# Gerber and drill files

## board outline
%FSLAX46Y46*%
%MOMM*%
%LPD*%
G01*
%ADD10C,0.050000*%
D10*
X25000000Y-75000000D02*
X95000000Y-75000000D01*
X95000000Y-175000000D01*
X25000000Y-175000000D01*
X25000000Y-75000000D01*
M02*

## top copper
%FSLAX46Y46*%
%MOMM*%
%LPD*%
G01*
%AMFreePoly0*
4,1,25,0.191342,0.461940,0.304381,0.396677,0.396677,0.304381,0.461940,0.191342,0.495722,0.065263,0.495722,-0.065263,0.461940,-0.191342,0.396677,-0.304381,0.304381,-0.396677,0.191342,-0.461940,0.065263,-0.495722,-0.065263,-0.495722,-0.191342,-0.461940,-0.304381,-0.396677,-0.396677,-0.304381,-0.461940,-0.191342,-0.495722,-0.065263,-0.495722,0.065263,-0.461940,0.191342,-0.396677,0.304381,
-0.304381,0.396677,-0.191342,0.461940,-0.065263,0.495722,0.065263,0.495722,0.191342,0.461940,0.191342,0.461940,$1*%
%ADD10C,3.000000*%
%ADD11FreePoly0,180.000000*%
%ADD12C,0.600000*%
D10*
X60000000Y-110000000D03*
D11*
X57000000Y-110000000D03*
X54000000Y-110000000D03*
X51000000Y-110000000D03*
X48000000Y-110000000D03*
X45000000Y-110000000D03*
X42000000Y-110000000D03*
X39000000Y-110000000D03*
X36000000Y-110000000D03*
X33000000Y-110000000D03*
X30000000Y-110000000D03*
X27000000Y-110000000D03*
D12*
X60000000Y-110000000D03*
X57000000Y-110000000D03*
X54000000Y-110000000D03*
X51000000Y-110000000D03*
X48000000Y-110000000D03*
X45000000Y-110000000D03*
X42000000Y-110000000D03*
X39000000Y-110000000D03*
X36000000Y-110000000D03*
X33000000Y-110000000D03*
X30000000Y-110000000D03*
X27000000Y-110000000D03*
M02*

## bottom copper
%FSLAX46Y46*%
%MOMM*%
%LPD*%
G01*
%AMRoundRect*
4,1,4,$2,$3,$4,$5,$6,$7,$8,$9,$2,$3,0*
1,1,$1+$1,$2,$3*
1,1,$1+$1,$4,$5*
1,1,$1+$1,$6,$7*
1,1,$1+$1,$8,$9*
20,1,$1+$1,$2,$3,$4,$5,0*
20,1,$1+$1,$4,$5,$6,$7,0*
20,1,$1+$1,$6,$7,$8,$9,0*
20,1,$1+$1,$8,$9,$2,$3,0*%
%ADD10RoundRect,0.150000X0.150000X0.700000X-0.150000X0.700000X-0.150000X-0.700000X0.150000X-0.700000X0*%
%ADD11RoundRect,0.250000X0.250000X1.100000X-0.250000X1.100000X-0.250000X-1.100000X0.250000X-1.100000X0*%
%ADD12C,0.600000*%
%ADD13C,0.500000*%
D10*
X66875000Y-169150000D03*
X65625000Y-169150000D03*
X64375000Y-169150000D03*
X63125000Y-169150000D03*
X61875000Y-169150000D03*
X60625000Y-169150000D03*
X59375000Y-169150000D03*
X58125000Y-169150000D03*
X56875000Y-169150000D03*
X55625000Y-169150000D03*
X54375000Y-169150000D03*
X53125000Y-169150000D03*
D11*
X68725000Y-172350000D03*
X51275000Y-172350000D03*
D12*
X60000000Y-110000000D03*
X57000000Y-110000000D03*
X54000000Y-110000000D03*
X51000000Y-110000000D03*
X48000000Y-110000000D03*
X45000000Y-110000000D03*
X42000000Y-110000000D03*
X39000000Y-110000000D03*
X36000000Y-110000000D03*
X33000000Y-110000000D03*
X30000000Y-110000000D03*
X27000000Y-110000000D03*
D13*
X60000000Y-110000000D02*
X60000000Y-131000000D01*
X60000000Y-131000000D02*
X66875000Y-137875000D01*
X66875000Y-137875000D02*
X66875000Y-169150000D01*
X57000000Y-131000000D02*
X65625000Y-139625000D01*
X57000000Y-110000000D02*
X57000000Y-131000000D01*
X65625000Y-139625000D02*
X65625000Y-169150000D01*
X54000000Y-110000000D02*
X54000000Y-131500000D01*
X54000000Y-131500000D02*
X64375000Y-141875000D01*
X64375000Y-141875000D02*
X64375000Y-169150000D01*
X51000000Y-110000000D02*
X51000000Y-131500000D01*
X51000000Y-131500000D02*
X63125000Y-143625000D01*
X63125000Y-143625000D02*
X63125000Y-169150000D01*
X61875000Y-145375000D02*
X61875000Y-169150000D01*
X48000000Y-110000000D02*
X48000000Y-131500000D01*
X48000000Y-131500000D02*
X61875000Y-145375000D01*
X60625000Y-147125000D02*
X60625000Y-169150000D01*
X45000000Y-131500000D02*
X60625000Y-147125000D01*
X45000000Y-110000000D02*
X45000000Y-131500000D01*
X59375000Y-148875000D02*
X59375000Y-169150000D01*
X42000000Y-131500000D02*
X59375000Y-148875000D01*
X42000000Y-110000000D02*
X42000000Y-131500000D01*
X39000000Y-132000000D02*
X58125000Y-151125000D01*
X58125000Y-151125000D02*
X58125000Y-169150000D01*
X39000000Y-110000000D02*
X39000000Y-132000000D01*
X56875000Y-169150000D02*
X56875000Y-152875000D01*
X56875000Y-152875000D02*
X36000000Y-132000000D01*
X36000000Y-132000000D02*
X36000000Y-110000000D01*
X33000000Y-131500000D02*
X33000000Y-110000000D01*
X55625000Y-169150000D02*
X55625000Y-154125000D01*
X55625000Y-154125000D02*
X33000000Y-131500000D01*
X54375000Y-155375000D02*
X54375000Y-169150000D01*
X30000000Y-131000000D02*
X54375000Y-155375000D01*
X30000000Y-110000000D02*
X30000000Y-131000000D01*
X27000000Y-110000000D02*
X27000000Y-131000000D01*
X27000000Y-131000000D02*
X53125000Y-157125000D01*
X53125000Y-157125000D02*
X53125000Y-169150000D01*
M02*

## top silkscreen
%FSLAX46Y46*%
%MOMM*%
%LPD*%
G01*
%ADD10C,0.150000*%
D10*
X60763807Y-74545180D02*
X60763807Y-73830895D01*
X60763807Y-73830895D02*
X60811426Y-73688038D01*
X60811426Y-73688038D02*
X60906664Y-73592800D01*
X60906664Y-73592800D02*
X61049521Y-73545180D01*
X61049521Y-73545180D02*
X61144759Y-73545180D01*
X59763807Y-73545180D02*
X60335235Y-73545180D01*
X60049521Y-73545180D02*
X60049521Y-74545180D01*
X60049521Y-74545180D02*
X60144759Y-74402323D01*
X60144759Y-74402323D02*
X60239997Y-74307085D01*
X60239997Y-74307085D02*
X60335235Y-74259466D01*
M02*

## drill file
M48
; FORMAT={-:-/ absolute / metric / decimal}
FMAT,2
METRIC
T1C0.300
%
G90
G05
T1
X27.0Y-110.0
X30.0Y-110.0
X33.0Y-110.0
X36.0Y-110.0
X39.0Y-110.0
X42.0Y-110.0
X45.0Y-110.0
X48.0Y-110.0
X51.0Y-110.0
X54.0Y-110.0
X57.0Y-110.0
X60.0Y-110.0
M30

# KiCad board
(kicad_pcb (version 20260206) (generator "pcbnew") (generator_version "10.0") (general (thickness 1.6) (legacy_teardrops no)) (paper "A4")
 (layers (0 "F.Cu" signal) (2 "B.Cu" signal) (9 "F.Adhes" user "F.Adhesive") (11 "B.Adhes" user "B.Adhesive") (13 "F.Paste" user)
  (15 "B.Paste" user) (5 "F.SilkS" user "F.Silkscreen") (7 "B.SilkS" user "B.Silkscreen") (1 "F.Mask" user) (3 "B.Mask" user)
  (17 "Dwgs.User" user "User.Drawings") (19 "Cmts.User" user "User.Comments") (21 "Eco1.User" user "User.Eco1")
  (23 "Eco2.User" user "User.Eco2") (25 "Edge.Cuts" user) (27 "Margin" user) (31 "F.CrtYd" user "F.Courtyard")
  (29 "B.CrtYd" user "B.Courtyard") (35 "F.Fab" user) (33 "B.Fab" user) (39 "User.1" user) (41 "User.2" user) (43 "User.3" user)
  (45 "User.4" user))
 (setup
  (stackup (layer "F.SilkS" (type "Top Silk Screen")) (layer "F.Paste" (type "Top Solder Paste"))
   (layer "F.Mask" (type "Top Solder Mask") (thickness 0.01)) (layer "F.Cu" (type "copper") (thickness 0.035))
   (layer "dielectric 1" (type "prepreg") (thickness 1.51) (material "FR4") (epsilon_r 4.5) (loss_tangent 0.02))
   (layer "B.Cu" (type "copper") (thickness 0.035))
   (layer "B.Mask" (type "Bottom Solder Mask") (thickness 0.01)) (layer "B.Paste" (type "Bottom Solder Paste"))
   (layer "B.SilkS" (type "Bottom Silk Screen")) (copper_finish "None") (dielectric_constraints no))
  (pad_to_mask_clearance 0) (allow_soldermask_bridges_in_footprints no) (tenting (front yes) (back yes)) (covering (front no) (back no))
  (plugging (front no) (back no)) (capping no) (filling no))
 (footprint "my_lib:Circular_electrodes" (layer "F.Cu") (at 60 110 180)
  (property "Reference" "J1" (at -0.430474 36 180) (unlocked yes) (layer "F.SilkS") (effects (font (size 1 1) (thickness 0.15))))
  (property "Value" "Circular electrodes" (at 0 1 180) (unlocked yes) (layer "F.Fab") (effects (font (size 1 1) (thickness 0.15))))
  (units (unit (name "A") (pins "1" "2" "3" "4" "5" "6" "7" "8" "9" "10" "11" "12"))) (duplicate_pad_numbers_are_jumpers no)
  (pad "1" smd circle (at 0 0 180) (size 3 3) (layers "F.Cu" "F.Mask" "F.Paste") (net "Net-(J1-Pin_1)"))
  (pad "2" smd custom (at 3 0 180) (size 1 1) (layers "F.Cu" "F.Mask" "F.Paste") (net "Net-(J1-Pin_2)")
   (options (clearance outline) (anchor circle)) (primitives))
  (pad "3" smd custom (at 6 0 180) (size 1 1) (layers "F.Cu" "F.Mask" "F.Paste") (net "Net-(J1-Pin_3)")
   (options (clearance outline) (anchor circle)) (primitives))
  (pad "4" smd custom (at 9 0 180) (size 1 1) (layers "F.Cu" "F.Mask" "F.Paste") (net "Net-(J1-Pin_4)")
   (options (clearance outline) (anchor circle)) (primitives))
  (pad "5" smd custom (at 12 0 180) (size 1 1) (layers "F.Cu" "F.Mask" "F.Paste") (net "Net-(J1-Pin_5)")
   (options (clearance outline) (anchor circle)) (primitives))
  (pad "6" smd custom (at 15 0 180) (size 1 1) (layers "F.Cu" "F.Mask" "F.Paste") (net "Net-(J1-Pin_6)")
   (options (clearance outline) (anchor circle)) (primitives))
  (pad "7" smd custom (at 18 0 180) (size 1 1) (layers "F.Cu" "F.Mask" "F.Paste") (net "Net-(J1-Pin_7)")
   (options (clearance outline) (anchor circle)) (primitives))
  (pad "8" smd custom (at 21 0 180) (size 1 1) (layers "F.Cu" "F.Mask" "F.Paste") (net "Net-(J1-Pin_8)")
   (options (clearance outline) (anchor circle)) (primitives))
  (pad "9" smd custom (at 24 0 180) (size 1 1) (layers "F.Cu" "F.Mask" "F.Paste") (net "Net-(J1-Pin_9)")
   (options (clearance outline) (anchor circle)) (primitives))
  (pad "10" smd custom (at 27 0 180) (size 1 1) (layers "F.Cu" "F.Mask" "F.Paste") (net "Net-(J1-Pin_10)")
   (options (clearance outline) (anchor circle)) (primitives))
  (pad "11" smd custom (at 30 0 180) (size 1 1) (layers "F.Cu" "F.Mask" "F.Paste") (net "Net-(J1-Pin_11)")
   (options (clearance outline) (anchor circle)) (primitives))
  (pad "12" smd custom (at 33 0 180) (size 1 1) (layers "F.Cu" "F.Mask" "F.Paste") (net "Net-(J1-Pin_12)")
   (options (clearance outline) (anchor circle)) (primitives)))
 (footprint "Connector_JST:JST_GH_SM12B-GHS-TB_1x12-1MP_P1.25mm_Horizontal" (layer "B.Cu") (at 60 171 180)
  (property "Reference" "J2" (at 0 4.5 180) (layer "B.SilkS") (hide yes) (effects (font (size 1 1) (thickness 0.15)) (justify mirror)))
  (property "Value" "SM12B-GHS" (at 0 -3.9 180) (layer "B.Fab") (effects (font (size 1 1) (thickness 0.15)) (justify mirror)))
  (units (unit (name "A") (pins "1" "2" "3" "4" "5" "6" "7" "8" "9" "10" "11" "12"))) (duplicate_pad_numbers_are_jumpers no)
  (pad "1" smd roundrect (at -6.875 1.85 180) (size 0.6 1.7) (layers "B.Cu" "B.Mask" "B.Paste") (roundrect_rratio 0.25)
   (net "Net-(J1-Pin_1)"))
  (pad "2" smd roundrect (at -5.625 1.85 180) (size 0.6 1.7) (layers "B.Cu" "B.Mask" "B.Paste") (roundrect_rratio 0.25)
   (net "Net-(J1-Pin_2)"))
  (pad "3" smd roundrect (at -4.375 1.85 180) (size 0.6 1.7) (layers "B.Cu" "B.Mask" "B.Paste") (roundrect_rratio 0.25)
   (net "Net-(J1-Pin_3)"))
  (pad "4" smd roundrect (at -3.125 1.85 180) (size 0.6 1.7) (layers "B.Cu" "B.Mask" "B.Paste") (roundrect_rratio 0.25)
   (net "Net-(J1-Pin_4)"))
  (pad "5" smd roundrect (at -1.875 1.85 180) (size 0.6 1.7) (layers "B.Cu" "B.Mask" "B.Paste") (roundrect_rratio 0.25)
   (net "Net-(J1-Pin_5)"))
  (pad "6" smd roundrect (at -0.625 1.85 180) (size 0.6 1.7) (layers "B.Cu" "B.Mask" "B.Paste") (roundrect_rratio 0.25)
   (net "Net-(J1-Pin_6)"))
  (pad "7" smd roundrect (at 0.625 1.85 180) (size 0.6 1.7) (layers "B.Cu" "B.Mask" "B.Paste") (roundrect_rratio 0.25)
   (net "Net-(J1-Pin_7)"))
  (pad "8" smd roundrect (at 1.875 1.85 180) (size 0.6 1.7) (layers "B.Cu" "B.Mask" "B.Paste") (roundrect_rratio 0.25)
   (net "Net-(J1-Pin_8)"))
  (pad "9" smd roundrect (at 3.125 1.85 180) (size 0.6 1.7) (layers "B.Cu" "B.Mask" "B.Paste") (roundrect_rratio 0.25)
   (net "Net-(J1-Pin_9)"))
  (pad "10" smd roundrect (at 4.375 1.85 180) (size 0.6 1.7) (layers "B.Cu" "B.Mask" "B.Paste") (roundrect_rratio 0.25)
   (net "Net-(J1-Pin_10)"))
  (pad "11" smd roundrect (at 5.625 1.85 180) (size 0.6 1.7) (layers "B.Cu" "B.Mask" "B.Paste") (roundrect_rratio 0.25)
   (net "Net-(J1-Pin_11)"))
  (pad "12" smd roundrect (at 6.875 1.85 180) (size 0.6 1.7) (layers "B.Cu" "B.Mask" "B.Paste") (roundrect_rratio 0.25)
   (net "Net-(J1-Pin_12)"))
  (pad "MP" smd roundrect (at -8.725 -1.35 180) (size 1 2.7) (layers "B.Cu" "B.Mask" "B.Paste") (roundrect_rratio 0.25))
  (pad "MP" smd roundrect (at 8.725 -1.35 180) (size 1 2.7) (layers "B.Cu" "B.Mask" "B.Paste") (roundrect_rratio 0.25)))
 (gr_rect (start 25 75) (end 95 175) (stroke (width 0.05) (type default)) (fill no) (layer "Edge.Cuts"))
 (via (at 60 110) (size 0.6) (drill 0.3) (layers "F.Cu" "B.Cu") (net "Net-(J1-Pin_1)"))
 (segment (start 60 110) (end 60 131) (width 0.5) (layer "B.Cu") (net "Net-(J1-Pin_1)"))
 (segment (start 60 131) (end 66.875 137.875) (width 0.5) (layer "B.Cu") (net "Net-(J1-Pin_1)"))
 (segment (start 66.875 137.875) (end 66.875 169.15) (width 0.5) (layer "B.Cu") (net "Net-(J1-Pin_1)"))
 (via (at 57 110) (size 0.6) (drill 0.3) (layers "F.Cu" "B.Cu") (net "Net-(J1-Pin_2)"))
 (segment (start 57 131) (end 65.625 139.625) (width 0.5) (layer "B.Cu") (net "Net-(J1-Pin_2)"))
 (segment (start 57 110) (end 57 131) (width 0.5) (layer "B.Cu") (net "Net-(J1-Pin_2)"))
 (segment (start 65.625 139.625) (end 65.625 169.15) (width 0.5) (layer "B.Cu") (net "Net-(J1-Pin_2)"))
 (via (at 54 110) (size 0.6) (drill 0.3) (layers "F.Cu" "B.Cu") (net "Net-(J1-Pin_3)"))
 (segment (start 54 110) (end 54 131.5) (width 0.5) (layer "B.Cu") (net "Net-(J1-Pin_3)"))
 (segment (start 54 131.5) (end 64.375 141.875) (width 0.5) (layer "B.Cu") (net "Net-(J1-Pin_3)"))
 (segment (start 64.375 141.875) (end 64.375 169.15) (width 0.5) (layer "B.Cu") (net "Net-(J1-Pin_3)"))
 (via (at 51 110) (size 0.6) (drill 0.3) (layers "F.Cu" "B.Cu") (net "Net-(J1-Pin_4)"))
 (segment (start 51 110) (end 51 131.5) (width 0.5) (layer "B.Cu") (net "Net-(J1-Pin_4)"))
 (segment (start 51 131.5) (end 63.125 143.625) (width 0.5) (layer "B.Cu") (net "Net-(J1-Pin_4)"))
 (segment (start 63.125 143.625) (end 63.125 169.15) (width 0.5) (layer "B.Cu") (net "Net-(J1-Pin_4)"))
 (via (at 48 110) (size 0.6) (drill 0.3) (layers "F.Cu" "B.Cu") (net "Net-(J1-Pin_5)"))
 (segment (start 61.875 145.375) (end 61.875 169.15) (width 0.5) (layer "B.Cu") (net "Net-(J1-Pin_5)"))
 (segment (start 48 110) (end 48 131.5) (width 0.5) (layer "B.Cu") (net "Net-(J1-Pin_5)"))
 (segment (start 48 131.5) (end 61.875 145.375) (width 0.5) (layer "B.Cu") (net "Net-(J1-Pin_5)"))
 (via (at 45 110) (size 0.6) (drill 0.3) (layers "F.Cu" "B.Cu") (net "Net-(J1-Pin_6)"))
 (segment (start 60.625 147.125) (end 60.625 169.15) (width 0.5) (layer "B.Cu") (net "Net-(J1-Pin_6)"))
 (segment (start 45 131.5) (end 60.625 147.125) (width 0.5) (layer "B.Cu") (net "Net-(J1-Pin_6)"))
 (segment (start 45 110) (end 45 131.5) (width 0.5) (layer "B.Cu") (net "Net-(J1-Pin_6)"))
 (via (at 42 110) (size 0.6) (drill 0.3) (layers "F.Cu" "B.Cu") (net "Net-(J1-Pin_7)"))
 (segment (start 59.375 148.875) (end 59.375 169.15) (width 0.5) (layer "B.Cu") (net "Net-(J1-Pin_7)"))
 (segment (start 42 131.5) (end 59.375 148.875) (width 0.5) (layer "B.Cu") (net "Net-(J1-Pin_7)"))
 (segment (start 42 110) (end 42 131.5) (width 0.5) (layer "B.Cu") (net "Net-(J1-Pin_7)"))
 (via (at 39 110) (size 0.6) (drill 0.3) (layers "F.Cu" "B.Cu") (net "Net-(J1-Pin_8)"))
 (segment (start 39 132) (end 58.125 151.125) (width 0.5) (layer "B.Cu") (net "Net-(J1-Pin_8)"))
 (segment (start 58.125 151.125) (end 58.125 169.15) (width 0.5) (layer "B.Cu") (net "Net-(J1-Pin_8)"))
 (segment (start 39 110) (end 39 132) (width 0.5) (layer "B.Cu") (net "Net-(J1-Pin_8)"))
 (via (at 36 110) (size 0.6) (drill 0.3) (layers "F.Cu" "B.Cu") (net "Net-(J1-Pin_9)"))
 (segment (start 56.875 169.15) (end 56.875 152.875) (width 0.5) (layer "B.Cu") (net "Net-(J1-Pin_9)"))
 (segment (start 56.875 152.875) (end 36 132) (width 0.5) (layer "B.Cu") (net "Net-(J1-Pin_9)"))
 (segment (start 36 132) (end 36 110) (width 0.5) (layer "B.Cu") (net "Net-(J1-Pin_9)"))
 (via (at 33 110) (size 0.6) (drill 0.3) (layers "F.Cu" "B.Cu") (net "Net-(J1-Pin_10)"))
 (segment (start 33 131.5) (end 33 110) (width 0.5) (layer "B.Cu") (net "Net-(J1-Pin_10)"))
 (segment (start 55.625 169.15) (end 55.625 154.125) (width 0.5) (layer "B.Cu") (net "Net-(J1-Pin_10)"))
 (segment (start 55.625 154.125) (end 33 131.5) (width 0.5) (layer "B.Cu") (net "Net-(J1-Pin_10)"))
 (via (at 30 110) (size 0.6) (drill 0.3) (layers "F.Cu" "B.Cu") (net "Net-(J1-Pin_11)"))
 (segment (start 54.375 155.375) (end 54.375 169.15) (width 0.5) (layer "B.Cu") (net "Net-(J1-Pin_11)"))
 (segment (start 30 131) (end 54.375 155.375) (width 0.5) (layer "B.Cu") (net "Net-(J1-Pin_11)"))
 (segment (start 30 110) (end 30 131) (width 0.5) (layer "B.Cu") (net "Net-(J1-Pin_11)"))
 (via (at 27 110) (size 0.6) (drill 0.3) (layers "F.Cu" "B.Cu") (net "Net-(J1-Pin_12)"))
 (segment (start 27 110) (end 27 131) (width 0.5) (layer "B.Cu") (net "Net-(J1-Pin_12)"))
 (segment (start 27 131) (end 53.125 157.125) (width 0.5) (layer "B.Cu") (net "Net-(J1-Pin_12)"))
 (segment (start 53.125 157.125) (end 53.125 169.15) (width 0.5) (layer "B.Cu") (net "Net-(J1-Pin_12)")))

